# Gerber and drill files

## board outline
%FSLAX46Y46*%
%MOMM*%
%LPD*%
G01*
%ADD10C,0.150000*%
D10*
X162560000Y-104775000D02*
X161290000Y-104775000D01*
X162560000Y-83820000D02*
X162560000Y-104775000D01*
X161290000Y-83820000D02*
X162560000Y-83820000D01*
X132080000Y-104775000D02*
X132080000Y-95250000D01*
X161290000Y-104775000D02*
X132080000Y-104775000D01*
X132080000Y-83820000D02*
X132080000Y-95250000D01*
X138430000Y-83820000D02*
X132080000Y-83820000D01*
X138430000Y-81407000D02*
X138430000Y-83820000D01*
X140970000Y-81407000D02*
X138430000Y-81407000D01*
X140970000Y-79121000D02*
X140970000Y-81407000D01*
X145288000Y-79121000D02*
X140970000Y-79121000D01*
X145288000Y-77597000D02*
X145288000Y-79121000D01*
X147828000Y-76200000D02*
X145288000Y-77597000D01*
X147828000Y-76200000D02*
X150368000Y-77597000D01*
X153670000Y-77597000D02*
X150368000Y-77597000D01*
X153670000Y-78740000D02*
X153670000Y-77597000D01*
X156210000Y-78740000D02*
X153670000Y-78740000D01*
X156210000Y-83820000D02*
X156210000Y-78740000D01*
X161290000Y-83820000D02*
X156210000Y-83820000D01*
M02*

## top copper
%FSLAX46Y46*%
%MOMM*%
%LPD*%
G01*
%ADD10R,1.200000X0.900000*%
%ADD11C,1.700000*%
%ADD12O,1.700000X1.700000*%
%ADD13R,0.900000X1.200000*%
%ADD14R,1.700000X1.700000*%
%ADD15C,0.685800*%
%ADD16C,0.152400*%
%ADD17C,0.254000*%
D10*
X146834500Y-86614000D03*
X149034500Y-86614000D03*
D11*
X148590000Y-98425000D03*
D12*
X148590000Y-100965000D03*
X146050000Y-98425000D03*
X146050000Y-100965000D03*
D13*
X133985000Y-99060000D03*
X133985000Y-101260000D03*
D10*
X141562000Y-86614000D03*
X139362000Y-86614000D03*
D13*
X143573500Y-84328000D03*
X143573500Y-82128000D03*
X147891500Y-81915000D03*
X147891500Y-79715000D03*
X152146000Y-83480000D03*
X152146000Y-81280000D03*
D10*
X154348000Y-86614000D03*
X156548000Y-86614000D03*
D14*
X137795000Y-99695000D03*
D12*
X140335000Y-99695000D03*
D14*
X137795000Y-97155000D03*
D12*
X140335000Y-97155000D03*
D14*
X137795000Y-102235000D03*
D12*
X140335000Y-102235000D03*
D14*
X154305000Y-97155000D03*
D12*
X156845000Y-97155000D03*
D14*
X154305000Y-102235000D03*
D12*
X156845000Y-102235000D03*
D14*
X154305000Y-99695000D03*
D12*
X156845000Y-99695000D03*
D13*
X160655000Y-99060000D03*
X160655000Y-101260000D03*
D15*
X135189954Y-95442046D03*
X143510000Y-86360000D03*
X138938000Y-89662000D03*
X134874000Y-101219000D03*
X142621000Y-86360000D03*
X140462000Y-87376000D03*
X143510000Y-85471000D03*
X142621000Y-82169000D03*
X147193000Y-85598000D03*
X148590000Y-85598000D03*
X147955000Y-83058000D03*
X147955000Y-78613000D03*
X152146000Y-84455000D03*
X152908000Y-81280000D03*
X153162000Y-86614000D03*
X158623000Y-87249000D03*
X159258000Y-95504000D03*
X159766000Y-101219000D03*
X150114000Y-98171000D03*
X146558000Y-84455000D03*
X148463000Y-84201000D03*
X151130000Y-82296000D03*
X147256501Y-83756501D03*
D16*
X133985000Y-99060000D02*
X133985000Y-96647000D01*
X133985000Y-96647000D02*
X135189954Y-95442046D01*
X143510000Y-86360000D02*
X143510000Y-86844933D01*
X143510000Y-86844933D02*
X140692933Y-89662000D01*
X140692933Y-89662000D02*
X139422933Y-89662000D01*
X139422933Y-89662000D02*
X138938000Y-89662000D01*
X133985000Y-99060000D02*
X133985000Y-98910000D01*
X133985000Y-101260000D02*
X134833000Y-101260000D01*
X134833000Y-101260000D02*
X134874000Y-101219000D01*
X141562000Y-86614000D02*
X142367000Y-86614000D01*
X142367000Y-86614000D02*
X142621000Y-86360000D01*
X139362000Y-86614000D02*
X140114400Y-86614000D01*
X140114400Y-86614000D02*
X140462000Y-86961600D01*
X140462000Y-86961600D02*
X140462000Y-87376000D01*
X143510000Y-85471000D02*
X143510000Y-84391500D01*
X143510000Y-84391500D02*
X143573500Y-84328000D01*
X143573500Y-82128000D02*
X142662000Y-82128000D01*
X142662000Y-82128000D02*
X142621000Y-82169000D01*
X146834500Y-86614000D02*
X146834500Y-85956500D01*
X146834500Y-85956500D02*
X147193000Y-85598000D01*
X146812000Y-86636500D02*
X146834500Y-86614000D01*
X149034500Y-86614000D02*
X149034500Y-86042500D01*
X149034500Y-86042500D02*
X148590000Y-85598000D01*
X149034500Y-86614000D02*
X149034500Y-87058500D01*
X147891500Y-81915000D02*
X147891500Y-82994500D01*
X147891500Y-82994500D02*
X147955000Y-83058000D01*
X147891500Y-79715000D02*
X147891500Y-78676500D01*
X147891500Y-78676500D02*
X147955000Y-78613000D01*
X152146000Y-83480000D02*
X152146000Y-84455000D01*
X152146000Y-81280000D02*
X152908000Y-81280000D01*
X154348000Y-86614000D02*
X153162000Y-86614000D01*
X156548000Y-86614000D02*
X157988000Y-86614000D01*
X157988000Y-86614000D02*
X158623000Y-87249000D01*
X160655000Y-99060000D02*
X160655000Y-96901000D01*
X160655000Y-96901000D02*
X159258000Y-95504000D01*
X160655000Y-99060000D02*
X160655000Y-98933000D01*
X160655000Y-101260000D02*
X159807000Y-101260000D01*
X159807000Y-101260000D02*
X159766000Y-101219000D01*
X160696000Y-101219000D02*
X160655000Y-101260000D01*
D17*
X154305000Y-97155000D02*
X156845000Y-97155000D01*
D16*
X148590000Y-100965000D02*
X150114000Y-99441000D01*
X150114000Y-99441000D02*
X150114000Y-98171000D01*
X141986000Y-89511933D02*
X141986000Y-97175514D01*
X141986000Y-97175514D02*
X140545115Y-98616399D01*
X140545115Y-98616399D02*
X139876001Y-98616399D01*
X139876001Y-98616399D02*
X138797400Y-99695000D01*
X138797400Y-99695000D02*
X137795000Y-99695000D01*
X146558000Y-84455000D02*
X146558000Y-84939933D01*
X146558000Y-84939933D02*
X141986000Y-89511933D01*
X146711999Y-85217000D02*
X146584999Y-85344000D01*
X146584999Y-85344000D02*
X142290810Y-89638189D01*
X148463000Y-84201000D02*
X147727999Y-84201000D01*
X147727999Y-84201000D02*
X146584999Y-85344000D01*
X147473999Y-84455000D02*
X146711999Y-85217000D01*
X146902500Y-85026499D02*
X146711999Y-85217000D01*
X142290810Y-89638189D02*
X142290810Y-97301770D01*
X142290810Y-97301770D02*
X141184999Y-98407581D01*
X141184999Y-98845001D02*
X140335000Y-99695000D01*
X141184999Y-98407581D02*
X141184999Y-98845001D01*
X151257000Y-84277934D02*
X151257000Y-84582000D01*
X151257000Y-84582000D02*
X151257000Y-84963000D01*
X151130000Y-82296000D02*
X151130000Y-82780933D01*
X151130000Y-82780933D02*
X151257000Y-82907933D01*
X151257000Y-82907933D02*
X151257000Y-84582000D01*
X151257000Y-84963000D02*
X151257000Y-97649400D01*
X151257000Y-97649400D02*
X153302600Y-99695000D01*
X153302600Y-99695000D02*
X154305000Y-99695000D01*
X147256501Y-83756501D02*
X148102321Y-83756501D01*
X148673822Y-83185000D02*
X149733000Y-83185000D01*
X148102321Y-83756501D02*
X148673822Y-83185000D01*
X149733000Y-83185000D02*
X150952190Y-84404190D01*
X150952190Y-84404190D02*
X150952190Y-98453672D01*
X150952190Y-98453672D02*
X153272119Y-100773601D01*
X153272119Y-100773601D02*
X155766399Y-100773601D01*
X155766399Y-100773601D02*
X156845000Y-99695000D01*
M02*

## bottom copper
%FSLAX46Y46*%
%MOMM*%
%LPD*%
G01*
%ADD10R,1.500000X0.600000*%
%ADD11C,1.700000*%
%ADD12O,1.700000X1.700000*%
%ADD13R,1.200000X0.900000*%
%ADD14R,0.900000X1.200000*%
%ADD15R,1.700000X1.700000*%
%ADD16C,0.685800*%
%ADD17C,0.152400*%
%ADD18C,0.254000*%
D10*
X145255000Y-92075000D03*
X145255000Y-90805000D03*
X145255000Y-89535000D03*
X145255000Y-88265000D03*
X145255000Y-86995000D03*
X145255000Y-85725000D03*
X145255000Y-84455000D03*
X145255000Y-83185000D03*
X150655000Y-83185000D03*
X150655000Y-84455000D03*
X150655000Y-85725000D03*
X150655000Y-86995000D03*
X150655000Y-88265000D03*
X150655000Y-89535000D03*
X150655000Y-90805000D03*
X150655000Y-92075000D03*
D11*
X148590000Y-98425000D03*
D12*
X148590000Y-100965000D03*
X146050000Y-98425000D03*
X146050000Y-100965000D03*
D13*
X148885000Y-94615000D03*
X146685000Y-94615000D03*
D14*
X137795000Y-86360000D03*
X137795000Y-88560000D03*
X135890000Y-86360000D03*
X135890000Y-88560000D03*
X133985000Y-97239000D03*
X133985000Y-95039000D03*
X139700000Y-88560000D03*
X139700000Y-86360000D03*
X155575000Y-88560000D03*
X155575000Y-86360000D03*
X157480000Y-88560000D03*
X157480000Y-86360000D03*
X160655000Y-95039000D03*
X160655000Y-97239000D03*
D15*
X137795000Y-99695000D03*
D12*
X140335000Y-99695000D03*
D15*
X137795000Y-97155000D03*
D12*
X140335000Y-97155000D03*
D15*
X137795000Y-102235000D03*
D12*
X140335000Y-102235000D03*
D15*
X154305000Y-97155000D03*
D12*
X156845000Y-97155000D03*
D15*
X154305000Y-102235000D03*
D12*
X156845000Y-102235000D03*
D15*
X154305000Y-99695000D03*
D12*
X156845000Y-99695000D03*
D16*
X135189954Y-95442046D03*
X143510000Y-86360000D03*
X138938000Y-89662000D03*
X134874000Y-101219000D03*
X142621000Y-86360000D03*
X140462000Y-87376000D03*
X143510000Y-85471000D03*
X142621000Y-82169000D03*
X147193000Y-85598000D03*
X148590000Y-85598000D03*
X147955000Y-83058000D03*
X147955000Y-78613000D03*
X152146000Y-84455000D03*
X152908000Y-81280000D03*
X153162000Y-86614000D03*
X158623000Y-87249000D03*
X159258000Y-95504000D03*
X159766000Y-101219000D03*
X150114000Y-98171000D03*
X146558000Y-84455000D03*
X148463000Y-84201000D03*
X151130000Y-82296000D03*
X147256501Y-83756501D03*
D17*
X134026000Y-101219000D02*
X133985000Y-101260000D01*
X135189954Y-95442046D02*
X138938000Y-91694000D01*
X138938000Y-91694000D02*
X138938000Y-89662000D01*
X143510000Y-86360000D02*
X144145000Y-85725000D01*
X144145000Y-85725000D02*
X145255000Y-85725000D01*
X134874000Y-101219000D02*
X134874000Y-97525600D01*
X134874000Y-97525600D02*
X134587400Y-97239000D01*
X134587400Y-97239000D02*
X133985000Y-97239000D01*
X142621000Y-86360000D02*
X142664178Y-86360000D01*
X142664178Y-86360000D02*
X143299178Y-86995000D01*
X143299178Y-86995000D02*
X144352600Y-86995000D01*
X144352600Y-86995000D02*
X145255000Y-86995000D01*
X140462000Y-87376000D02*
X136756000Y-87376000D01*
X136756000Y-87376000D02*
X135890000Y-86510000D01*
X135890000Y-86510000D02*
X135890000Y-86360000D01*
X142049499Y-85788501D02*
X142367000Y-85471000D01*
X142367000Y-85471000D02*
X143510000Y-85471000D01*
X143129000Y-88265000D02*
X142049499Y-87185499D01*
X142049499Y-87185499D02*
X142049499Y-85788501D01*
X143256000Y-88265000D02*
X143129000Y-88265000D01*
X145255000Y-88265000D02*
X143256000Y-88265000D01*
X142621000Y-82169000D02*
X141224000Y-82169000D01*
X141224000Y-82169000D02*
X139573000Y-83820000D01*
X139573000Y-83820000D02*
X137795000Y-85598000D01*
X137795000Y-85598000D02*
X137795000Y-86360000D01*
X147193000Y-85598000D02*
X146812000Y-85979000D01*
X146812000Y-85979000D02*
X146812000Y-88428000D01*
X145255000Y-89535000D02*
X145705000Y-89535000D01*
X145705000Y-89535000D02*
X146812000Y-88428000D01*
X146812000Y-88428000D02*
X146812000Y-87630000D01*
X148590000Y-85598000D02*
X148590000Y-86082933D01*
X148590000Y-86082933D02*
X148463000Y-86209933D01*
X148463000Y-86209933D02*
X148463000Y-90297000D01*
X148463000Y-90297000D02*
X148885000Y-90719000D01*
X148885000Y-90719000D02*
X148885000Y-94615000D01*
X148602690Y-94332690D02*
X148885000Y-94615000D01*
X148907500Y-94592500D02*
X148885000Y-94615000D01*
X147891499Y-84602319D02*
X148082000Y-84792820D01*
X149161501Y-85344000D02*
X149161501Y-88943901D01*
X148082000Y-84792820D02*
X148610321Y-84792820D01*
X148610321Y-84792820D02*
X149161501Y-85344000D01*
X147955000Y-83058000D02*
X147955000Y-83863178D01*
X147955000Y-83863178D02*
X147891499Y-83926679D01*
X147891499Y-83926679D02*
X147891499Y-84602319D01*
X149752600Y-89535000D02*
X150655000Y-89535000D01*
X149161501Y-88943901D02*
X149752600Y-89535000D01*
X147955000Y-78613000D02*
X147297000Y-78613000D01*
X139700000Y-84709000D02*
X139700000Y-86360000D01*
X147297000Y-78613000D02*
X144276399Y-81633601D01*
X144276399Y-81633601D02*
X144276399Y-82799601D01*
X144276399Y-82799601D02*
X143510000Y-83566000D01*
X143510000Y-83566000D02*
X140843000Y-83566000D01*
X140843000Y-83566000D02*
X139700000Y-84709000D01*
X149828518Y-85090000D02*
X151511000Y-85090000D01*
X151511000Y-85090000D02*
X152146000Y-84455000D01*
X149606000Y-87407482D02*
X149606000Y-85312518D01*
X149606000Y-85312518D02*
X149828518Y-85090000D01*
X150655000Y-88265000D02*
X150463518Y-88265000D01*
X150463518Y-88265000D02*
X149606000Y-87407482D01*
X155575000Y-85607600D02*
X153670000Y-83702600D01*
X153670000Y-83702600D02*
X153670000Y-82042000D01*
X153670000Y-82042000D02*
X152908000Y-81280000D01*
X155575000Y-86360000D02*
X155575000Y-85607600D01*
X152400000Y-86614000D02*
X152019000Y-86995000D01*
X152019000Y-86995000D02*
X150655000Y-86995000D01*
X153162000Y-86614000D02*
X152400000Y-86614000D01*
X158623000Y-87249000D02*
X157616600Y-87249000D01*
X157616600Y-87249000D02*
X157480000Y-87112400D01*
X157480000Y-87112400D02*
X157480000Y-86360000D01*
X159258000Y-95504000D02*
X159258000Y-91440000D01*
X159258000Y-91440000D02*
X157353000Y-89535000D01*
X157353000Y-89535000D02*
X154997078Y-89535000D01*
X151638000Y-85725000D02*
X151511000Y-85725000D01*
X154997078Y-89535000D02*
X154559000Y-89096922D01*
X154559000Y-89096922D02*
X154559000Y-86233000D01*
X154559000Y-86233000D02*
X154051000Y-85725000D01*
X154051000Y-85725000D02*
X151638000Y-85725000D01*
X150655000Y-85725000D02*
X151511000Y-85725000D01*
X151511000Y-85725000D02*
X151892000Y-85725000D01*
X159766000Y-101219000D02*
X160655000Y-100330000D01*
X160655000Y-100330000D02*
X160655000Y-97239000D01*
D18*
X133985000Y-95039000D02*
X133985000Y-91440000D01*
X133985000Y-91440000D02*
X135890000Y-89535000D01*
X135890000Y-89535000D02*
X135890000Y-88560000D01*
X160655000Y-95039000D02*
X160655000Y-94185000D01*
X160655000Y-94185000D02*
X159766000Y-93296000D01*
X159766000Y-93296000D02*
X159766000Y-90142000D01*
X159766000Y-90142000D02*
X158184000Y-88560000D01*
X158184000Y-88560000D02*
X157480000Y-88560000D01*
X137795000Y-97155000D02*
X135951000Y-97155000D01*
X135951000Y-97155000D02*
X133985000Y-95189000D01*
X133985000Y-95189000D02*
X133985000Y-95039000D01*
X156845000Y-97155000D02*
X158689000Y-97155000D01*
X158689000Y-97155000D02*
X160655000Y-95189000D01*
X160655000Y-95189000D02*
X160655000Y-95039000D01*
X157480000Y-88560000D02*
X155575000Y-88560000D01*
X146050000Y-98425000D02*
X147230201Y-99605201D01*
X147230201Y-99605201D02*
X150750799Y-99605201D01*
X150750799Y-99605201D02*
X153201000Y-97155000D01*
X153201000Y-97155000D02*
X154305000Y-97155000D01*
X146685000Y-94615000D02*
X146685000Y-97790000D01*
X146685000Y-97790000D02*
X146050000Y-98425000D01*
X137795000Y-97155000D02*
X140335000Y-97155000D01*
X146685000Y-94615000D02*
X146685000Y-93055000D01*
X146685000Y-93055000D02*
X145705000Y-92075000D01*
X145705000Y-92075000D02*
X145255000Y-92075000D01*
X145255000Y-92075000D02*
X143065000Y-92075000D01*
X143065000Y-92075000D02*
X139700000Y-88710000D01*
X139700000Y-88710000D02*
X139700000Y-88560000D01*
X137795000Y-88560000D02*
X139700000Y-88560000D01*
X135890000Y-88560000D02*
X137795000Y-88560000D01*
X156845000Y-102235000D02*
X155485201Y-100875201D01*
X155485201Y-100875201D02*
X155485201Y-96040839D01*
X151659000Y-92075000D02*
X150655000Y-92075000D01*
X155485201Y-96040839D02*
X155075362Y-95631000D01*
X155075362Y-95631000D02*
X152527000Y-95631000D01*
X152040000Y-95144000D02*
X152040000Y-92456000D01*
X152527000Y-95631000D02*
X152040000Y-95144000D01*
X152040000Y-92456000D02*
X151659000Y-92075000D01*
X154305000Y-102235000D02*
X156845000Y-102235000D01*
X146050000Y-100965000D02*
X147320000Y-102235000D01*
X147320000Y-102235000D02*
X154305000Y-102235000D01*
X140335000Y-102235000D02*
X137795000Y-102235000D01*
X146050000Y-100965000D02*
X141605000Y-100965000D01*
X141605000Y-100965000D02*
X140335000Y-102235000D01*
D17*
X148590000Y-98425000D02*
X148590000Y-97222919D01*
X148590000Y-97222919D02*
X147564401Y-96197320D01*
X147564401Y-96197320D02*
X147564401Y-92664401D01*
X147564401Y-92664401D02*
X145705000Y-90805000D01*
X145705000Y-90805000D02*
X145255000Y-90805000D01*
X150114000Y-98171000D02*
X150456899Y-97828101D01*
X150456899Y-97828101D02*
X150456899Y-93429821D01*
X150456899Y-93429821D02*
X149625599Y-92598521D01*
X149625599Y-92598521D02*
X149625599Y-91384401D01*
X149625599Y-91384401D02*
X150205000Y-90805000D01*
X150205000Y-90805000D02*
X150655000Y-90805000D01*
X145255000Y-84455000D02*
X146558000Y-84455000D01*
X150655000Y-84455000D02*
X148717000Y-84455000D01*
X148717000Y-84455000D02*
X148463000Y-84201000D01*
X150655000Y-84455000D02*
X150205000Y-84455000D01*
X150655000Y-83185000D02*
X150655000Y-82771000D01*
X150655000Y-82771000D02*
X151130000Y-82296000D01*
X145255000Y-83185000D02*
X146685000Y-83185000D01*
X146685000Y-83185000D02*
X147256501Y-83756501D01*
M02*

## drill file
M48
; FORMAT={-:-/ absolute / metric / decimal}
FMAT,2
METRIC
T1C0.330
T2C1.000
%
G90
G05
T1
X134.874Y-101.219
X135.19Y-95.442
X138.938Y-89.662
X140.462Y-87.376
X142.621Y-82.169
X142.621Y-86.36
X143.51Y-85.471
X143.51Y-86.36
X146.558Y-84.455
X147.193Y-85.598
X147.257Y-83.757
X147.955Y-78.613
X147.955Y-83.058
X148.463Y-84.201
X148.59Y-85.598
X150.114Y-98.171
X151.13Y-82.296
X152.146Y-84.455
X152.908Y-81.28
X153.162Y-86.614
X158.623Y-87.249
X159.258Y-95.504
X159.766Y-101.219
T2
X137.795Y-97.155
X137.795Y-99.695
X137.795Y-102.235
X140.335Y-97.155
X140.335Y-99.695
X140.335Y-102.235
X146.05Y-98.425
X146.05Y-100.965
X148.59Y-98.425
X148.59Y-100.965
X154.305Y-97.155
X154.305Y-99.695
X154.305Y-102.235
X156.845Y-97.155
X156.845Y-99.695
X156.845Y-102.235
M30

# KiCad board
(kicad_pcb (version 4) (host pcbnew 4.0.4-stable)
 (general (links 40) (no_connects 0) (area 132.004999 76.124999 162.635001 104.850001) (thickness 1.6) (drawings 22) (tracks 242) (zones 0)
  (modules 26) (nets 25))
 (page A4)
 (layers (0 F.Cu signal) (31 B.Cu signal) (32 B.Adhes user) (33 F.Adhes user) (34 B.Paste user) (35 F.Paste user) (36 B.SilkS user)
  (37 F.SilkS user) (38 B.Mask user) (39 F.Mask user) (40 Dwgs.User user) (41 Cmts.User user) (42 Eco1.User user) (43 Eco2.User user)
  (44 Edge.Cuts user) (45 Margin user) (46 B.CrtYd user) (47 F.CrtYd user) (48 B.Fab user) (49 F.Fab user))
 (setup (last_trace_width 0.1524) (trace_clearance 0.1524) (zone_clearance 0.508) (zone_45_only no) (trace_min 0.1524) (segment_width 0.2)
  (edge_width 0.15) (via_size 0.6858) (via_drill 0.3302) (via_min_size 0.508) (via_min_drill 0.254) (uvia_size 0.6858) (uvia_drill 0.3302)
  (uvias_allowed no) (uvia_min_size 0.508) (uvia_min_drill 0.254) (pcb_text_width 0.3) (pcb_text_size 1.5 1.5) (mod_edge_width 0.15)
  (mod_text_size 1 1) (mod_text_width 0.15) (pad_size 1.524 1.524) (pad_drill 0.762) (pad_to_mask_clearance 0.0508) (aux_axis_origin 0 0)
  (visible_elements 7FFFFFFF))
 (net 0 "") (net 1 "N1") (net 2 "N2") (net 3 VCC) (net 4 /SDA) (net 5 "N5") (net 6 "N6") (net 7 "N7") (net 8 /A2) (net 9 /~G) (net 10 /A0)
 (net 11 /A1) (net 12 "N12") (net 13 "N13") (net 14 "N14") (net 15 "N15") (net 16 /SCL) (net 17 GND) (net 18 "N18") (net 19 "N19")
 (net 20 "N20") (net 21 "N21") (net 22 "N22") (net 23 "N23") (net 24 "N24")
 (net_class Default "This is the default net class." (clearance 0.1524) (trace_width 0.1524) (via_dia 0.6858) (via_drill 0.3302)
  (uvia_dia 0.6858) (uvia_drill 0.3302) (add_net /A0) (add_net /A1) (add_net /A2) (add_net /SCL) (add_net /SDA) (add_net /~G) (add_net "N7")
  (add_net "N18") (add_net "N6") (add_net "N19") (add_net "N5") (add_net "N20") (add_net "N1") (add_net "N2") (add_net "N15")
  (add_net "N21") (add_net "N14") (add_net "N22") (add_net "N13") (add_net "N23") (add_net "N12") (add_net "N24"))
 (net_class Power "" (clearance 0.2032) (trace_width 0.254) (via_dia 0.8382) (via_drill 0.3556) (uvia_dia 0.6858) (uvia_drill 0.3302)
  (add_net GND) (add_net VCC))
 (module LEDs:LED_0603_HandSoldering (layer F.Cu) (at 147.9345 86.614)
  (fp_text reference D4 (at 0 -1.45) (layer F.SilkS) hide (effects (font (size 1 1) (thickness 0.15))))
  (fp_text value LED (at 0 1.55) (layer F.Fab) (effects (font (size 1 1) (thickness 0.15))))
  (pad 1 smd rect (at -1.1 0) (size 1.2 0.9) (layers F.Cu F.Paste F.Mask) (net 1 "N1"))
  (pad 2 smd rect (at 1.1 0) (size 1.2 0.9) (layers F.Cu F.Paste F.Mask) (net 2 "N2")))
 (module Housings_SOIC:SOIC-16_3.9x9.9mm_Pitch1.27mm (layer B.Cu) (at 147.955 87.63)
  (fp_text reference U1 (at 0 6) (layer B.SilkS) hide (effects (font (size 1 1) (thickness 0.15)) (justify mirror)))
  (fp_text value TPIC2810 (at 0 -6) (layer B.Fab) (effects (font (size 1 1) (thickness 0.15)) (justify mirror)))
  (pad 1 smd rect (at -2.7 4.445) (size 1.5 0.6) (layers B.Cu B.Paste B.Mask) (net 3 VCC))
  (pad 2 smd rect (at -2.7 3.175) (size 1.5 0.6) (layers B.Cu B.Paste B.Mask) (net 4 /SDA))
  (pad 3 smd rect (at -2.7 1.905) (size 1.5 0.6) (layers B.Cu B.Paste B.Mask) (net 1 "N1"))
  (pad 4 smd rect (at -2.7 0.635) (size 1.5 0.6) (layers B.Cu B.Paste B.Mask) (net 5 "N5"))
  (pad 5 smd rect (at -2.7 -0.635) (size 1.5 0.6) (layers B.Cu B.Paste B.Mask) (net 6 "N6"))
  (pad 6 smd rect (at -2.7 -1.905) (size 1.5 0.6) (layers B.Cu B.Paste B.Mask) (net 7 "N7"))
  (pad 7 smd rect (at -2.7 -3.175) (size 1.5 0.6) (layers B.Cu B.Paste B.Mask) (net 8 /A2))
  (pad 8 smd rect (at -2.7 -4.445) (size 1.5 0.6) (layers B.Cu B.Paste B.Mask) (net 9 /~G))
  (pad 9 smd rect (at 2.7 -4.445) (size 1.5 0.6) (layers B.Cu B.Paste B.Mask) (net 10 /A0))
  (pad 10 smd rect (at 2.7 -3.175) (size 1.5 0.6) (layers B.Cu B.Paste B.Mask) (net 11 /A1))
  (pad 11 smd rect (at 2.7 -1.905) (size 1.5 0.6) (layers B.Cu B.Paste B.Mask) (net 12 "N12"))
  (pad 12 smd rect (at 2.7 -0.635) (size 1.5 0.6) (layers B.Cu B.Paste B.Mask) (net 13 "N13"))
  (pad 13 smd rect (at 2.7 0.635) (size 1.5 0.6) (layers B.Cu B.Paste B.Mask) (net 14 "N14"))
  (pad 14 smd rect (at 2.7 1.905) (size 1.5 0.6) (layers B.Cu B.Paste B.Mask) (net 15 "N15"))
  (pad 15 smd rect (at 2.7 3.175) (size 1.5 0.6) (layers B.Cu B.Paste B.Mask) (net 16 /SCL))
  (pad 16 smd rect (at 2.7 4.445) (size 1.5 0.6) (layers B.Cu B.Paste B.Mask) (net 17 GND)))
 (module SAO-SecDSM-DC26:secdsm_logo (layer F.Cu) (at 147.32 85.979)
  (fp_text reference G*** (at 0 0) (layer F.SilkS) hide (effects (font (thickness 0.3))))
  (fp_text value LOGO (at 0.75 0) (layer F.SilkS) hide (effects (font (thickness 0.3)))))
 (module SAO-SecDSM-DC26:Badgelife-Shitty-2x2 (layer F.Cu) (at 147.32 99.695)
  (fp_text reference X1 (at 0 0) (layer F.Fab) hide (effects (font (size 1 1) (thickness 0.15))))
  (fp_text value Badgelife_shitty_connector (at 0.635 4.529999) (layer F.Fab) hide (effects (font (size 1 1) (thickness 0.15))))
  (pad 4 thru_hole circle (at 1.27 -1.27) (size 1.7 1.7) (drill 1) (layers *.Cu *.Mask) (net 4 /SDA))
  (pad 3 thru_hole oval (at 1.27 1.27) (size 1.7 1.7) (drill 1) (layers *.Cu *.Mask) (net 16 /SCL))
  (pad 1 thru_hole oval (at -1.27 -1.27) (size 1.7 1.7) (drill 1) (layers *.Cu *.Mask) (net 3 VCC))
  (pad 2 thru_hole oval (at -1.27 1.27) (size 1.7 1.7) (drill 1) (layers *.Cu *.Mask) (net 17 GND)))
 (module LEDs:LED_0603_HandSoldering (layer F.Cu) (at 133.985 100.16 270)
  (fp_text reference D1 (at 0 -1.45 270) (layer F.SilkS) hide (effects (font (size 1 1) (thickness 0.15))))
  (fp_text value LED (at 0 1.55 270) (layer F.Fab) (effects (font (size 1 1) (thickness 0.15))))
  (pad 1 smd rect (at -1.1 0 270) (size 1.2 0.9) (layers F.Cu F.Paste F.Mask) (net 7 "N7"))
  (pad 2 smd rect (at 1.1 0 270) (size 1.2 0.9) (layers F.Cu F.Paste F.Mask) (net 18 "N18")))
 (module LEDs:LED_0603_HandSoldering (layer F.Cu) (at 140.462 86.614 180)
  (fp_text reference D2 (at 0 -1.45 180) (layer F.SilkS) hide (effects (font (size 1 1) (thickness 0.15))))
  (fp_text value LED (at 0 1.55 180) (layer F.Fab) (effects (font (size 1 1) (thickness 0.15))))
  (pad 1 smd rect (at -1.1 0 180) (size 1.2 0.9) (layers F.Cu F.Paste F.Mask) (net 6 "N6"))
  (pad 2 smd rect (at 1.1 0 180) (size 1.2 0.9) (layers F.Cu F.Paste F.Mask) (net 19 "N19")))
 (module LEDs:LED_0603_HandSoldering (layer F.Cu) (at 143.5735 83.228 90)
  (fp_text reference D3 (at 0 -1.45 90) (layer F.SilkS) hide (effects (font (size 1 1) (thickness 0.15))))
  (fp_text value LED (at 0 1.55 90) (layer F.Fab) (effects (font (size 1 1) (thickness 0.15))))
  (pad 1 smd rect (at -1.1 0 90) (size 1.2 0.9) (layers F.Cu F.Paste F.Mask) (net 5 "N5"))
  (pad 2 smd rect (at 1.1 0 90) (size 1.2 0.9) (layers F.Cu F.Paste F.Mask) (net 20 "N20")))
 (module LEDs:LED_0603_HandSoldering (layer F.Cu) (at 147.8915 80.815 90)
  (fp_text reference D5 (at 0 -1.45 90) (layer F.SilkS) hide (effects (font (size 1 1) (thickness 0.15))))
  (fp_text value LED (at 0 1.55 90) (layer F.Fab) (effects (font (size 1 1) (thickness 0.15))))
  (pad 1 smd rect (at -1.1 0 90) (size 1.2 0.9) (layers F.Cu F.Paste F.Mask) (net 15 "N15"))
  (pad 2 smd rect (at 1.1 0 90) (size 1.2 0.9) (layers F.Cu F.Paste F.Mask) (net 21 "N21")))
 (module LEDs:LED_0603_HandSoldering (layer F.Cu) (at 152.146 82.38 90)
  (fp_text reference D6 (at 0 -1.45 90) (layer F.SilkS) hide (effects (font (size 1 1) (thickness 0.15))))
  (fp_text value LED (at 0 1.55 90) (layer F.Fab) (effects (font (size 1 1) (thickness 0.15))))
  (pad 1 smd rect (at -1.1 0 90) (size 1.2 0.9) (layers F.Cu F.Paste F.Mask) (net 14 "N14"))
  (pad 2 smd rect (at 1.1 0 90) (size 1.2 0.9) (layers F.Cu F.Paste F.Mask) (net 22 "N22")))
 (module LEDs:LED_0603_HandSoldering (layer F.Cu) (at 155.448 86.614)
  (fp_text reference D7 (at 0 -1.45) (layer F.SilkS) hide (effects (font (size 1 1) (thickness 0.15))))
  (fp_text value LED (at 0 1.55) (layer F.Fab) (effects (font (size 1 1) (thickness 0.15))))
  (pad 1 smd rect (at -1.1 0) (size 1.2 0.9) (layers F.Cu F.Paste F.Mask) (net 13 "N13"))
  (pad 2 smd rect (at 1.1 0) (size 1.2 0.9) (layers F.Cu F.Paste F.Mask) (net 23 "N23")))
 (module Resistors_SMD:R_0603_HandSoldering (layer B.Cu) (at 147.785 94.615 180)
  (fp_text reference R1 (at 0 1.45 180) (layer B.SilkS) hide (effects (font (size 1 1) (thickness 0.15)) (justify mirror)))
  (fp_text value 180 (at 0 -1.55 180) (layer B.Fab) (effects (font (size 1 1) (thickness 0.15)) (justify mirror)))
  (pad 1 smd rect (at -1.1 0 180) (size 1.2 0.9) (layers B.Cu B.Paste B.Mask) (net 2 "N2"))
  (pad 2 smd rect (at 1.1 0 180) (size 1.2 0.9) (layers B.Cu B.Paste B.Mask) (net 3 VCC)))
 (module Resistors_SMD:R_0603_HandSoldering (layer B.Cu) (at 137.795 87.46 270)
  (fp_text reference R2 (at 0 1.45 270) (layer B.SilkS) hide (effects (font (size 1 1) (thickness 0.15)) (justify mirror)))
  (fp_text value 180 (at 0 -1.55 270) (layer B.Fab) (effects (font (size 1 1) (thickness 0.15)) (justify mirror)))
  (pad 1 smd rect (at -1.1 0 270) (size 1.2 0.9) (layers B.Cu B.Paste B.Mask) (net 20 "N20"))
  (pad 2 smd rect (at 1.1 0 270) (size 1.2 0.9) (layers B.Cu B.Paste B.Mask) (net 3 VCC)))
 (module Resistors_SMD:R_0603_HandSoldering (layer B.Cu) (at 135.89 87.46 270)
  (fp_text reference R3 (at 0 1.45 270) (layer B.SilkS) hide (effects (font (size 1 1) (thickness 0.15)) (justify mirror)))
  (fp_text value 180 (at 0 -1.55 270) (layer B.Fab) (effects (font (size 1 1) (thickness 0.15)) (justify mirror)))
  (pad 1 smd rect (at -1.1 0 270) (size 1.2 0.9) (layers B.Cu B.Paste B.Mask) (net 19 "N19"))
  (pad 2 smd rect (at 1.1 0 270) (size 1.2 0.9) (layers B.Cu B.Paste B.Mask) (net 3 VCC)))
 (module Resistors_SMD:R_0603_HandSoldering (layer B.Cu) (at 133.985 96.139 90)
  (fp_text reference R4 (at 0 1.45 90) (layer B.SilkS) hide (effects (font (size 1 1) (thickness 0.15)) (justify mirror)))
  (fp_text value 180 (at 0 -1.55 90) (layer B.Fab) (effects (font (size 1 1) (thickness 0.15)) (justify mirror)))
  (pad 1 smd rect (at -1.1 0 90) (size 1.2 0.9) (layers B.Cu B.Paste B.Mask) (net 18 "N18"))
  (pad 2 smd rect (at 1.1 0 90) (size 1.2 0.9) (layers B.Cu B.Paste B.Mask) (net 3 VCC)))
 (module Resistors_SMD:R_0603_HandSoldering (layer B.Cu) (at 139.7 87.46 90)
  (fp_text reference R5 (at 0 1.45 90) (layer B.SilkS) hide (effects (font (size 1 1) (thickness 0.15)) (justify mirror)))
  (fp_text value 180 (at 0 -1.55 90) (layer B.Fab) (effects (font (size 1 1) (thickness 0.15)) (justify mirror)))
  (pad 1 smd rect (at -1.1 0 90) (size 1.2 0.9) (layers B.Cu B.Paste B.Mask) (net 3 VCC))
  (pad 2 smd rect (at 1.1 0 90) (size 1.2 0.9) (layers B.Cu B.Paste B.Mask) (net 21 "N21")))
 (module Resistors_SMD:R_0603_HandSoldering (layer B.Cu) (at 155.575 87.46 90)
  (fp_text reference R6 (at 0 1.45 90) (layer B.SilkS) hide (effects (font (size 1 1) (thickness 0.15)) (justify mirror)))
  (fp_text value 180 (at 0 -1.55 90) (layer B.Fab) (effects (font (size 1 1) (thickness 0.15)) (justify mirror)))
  (pad 1 smd rect (at -1.1 0 90) (size 1.2 0.9) (layers B.Cu B.Paste B.Mask) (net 3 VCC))
  (pad 2 smd rect (at 1.1 0 90) (size 1.2 0.9) (layers B.Cu B.Paste B.Mask) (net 22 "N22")))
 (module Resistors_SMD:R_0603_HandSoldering (layer B.Cu) (at 157.48 87.46 90)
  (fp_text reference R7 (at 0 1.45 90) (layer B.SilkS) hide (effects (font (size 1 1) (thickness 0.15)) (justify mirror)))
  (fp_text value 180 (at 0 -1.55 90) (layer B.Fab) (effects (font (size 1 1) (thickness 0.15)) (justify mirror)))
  (pad 1 smd rect (at -1.1 0 90) (size 1.2 0.9) (layers B.Cu B.Paste B.Mask) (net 3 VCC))
  (pad 2 smd rect (at 1.1 0 90) (size 1.2 0.9) (layers B.Cu B.Paste B.Mask) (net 23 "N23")))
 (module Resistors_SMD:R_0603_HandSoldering (layer B.Cu) (at 160.655 96.139 270)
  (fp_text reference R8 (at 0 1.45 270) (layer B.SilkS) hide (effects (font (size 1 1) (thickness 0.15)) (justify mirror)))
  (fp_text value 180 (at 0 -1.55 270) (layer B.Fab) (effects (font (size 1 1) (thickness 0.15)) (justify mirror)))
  (pad 1 smd rect (at -1.1 0 270) (size 1.2 0.9) (layers B.Cu B.Paste B.Mask) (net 3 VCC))
  (pad 2 smd rect (at 1.1 0 270) (size 1.2 0.9) (layers B.Cu B.Paste B.Mask) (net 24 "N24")))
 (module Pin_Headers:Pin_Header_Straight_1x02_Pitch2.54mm (layer F.Cu) (at 137.795 99.695 90)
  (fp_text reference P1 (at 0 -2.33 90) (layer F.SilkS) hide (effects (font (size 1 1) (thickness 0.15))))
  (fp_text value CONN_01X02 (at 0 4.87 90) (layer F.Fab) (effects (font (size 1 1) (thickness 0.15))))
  (pad 1 thru_hole rect (at 0 0 90) (size 1.7 1.7) (drill 1) (layers *.Cu *.Mask) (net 8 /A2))
  (pad 2 thru_hole oval (at 0 2.54 90) (size 1.7 1.7) (drill 1) (layers *.Cu *.Mask) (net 11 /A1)))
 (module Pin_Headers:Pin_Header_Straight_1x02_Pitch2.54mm (layer F.Cu) (at 137.795 97.155 90)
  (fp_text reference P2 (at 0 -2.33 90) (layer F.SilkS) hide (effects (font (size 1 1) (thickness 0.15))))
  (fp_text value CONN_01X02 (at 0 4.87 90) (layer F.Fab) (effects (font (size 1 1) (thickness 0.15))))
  (pad 1 thru_hole rect (at 0 0 90) (size 1.7 1.7) (drill 1) (layers *.Cu *.Mask) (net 3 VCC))
  (pad 2 thru_hole oval (at 0 2.54 90) (size 1.7 1.7) (drill 1) (layers *.Cu *.Mask) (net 3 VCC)))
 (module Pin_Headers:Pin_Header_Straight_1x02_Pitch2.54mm (layer F.Cu) (at 137.795 102.235 90)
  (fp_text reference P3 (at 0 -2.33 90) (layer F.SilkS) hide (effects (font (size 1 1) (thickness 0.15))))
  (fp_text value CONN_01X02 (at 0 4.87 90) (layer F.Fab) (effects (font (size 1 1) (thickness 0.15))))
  (pad 1 thru_hole rect (at 0 0 90) (size 1.7 1.7) (drill 1) (layers *.Cu *.Mask) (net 17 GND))
  (pad 2 thru_hole oval (at 0 2.54 90) (size 1.7 1.7) (drill 1) (layers *.Cu *.Mask) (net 17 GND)))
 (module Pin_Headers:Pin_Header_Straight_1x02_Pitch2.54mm (layer F.Cu) (at 154.305 97.155 90)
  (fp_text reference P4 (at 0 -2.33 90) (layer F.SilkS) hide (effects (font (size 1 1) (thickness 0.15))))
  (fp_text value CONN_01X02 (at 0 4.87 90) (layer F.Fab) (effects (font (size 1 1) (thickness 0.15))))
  (pad 1 thru_hole rect (at 0 0 90) (size 1.7 1.7) (drill 1) (layers *.Cu *.Mask) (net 3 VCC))
  (pad 2 thru_hole oval (at 0 2.54 90) (size 1.7 1.7) (drill 1) (layers *.Cu *.Mask) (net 3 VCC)))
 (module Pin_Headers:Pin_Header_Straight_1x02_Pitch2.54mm (layer F.Cu) (at 154.305 102.235 90)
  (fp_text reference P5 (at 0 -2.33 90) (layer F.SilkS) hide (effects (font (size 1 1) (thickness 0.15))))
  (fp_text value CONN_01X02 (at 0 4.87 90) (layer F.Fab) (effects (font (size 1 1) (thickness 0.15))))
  (pad 1 thru_hole rect (at 0 0 90) (size 1.7 1.7) (drill 1) (layers *.Cu *.Mask) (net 17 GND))
  (pad 2 thru_hole oval (at 0 2.54 90) (size 1.7 1.7) (drill 1) (layers *.Cu *.Mask) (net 17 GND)))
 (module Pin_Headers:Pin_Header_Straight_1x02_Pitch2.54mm (layer F.Cu) (at 154.305 99.695 90)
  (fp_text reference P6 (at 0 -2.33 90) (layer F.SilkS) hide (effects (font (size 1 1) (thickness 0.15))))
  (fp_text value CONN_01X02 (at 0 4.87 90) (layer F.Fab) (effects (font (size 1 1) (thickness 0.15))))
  (pad 1 thru_hole rect (at 0 0 90) (size 1.7 1.7) (drill 1) (layers *.Cu *.Mask) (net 10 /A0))
  (pad 2 thru_hole oval (at 0 2.54 90) (size 1.7 1.7) (drill 1) (layers *.Cu *.Mask) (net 9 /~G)))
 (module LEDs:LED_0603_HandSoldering (layer F.Cu) (at 160.655 100.16 270)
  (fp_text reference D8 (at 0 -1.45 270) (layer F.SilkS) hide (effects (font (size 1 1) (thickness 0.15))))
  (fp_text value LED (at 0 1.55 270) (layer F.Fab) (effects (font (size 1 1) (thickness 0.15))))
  (pad 1 smd rect (at -1.1 0 270) (size 1.2 0.9) (layers F.Cu F.Paste F.Mask) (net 12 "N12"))
  (pad 2 smd rect (at 1.1 0 270) (size 1.2 0.9) (layers F.Cu F.Paste F.Mask) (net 24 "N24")))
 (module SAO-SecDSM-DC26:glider (layer B.Cu) (at 155.575 92.583 180)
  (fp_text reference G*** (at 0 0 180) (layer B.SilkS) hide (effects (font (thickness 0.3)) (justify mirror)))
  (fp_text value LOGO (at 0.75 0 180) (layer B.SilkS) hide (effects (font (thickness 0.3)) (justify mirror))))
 (gr_line (start 162.56 104.775) (end 161.29 104.775) (layer Edge.Cuts) (width 0.15))
 (gr_line (start 162.56 83.82) (end 162.56 104.775) (layer Edge.Cuts) (width 0.15))
 (gr_line (start 161.29 83.82) (end 162.56 83.82) (layer Edge.Cuts) (width 0.15))
 (gr_line (start 132.08 104.775) (end 132.08 95.25) (layer Edge.Cuts) (width 0.15))
 (gr_line (start 161.29 104.775) (end 132.08 104.775) (layer Edge.Cuts) (width 0.15))
 (gr_line (start 132.08 83.82) (end 132.08 95.25) (layer Edge.Cuts) (width 0.15))
 (gr_line (start 138.43 83.82) (end 132.08 83.82) (layer Edge.Cuts) (width 0.15))
 (gr_line (start 138.43 81.407) (end 138.43 83.82) (layer Edge.Cuts) (width 0.15))
 (gr_line (start 140.97 81.407) (end 138.43 81.407) (layer Edge.Cuts) (width 0.15))
 (gr_line (start 140.97 79.121) (end 140.97 81.407) (layer Edge.Cuts) (width 0.15))
 (gr_line (start 145.288 79.121) (end 140.97 79.121) (layer Edge.Cuts) (width 0.15))
 (gr_line (start 145.288 77.597) (end 145.288 79.121) (layer Edge.Cuts) (width 0.15))
 (gr_line (start 147.828 76.2) (end 145.288 77.597) (layer Edge.Cuts) (width 0.15))
 (gr_line (start 147.828 76.2) (end 150.368 77.597) (layer Edge.Cuts) (width 0.15))
 (gr_line (start 153.67 77.597) (end 150.368 77.597) (layer Edge.Cuts) (width 0.15))
 (gr_line (start 153.67 78.74) (end 153.67 77.597) (layer Edge.Cuts) (width 0.15))
 (gr_line (start 156.21 78.74) (end 153.67 78.74) (layer Edge.Cuts) (width 0.15))
 (gr_line (start 156.21 83.82) (end 156.21 78.74) (layer Edge.Cuts) (width 0.15))
 (gr_line (start 161.29 83.82) (end 156.21 83.82) (layer Edge.Cuts) (width 0.15))
 (segment (start 134.026 101.219) (end 133.985 101.26) (width 0.1524) (layer B.Cu) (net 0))
 (segment (start 135.189954 95.442046) (end 138.938 91.694) (width 0.1524) (layer B.Cu) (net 7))
 (segment (start 138.938 91.694) (end 138.938 89.662) (width 0.1524) (layer B.Cu) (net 7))
 (segment (start 133.985 99.06) (end 133.985 96.647) (width 0.1524) (layer F.Cu) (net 7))
 (segment (start 133.985 96.647) (end 135.189954 95.442046) (width 0.1524) (layer F.Cu) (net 7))
 (via (at 135.189954 95.442046) (size 0.6858) (drill 0.3302) (layers F.Cu B.Cu) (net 7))
 (segment (start 143.51 86.36) (end 143.51 86.844933) (width 0.1524) (layer F.Cu) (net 7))
 (segment (start 143.51 86.844933) (end 140.692933 89.662) (width 0.1524) (layer F.Cu) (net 7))
 (segment (start 140.692933 89.662) (end 139.422933 89.662) (width 0.1524) (layer F.Cu) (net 7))
 (segment (start 139.422933 89.662) (end 138.938 89.662) (width 0.1524) (layer F.Cu) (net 7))
 (segment (start 143.51 86.36) (end 144.145 85.725) (width 0.1524) (layer B.Cu) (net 7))
 (segment (start 144.145 85.725) (end 145.255 85.725) (width 0.1524) (layer B.Cu) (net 7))
 (via (at 143.51 86.36) (size 0.6858) (drill 0.3302) (layers F.Cu B.Cu) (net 7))
 (via (at 138.938 89.662) (size 0.6858) (drill 0.3302) (layers F.Cu B.Cu) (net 7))
 (segment (start 133.985 99.06) (end 133.985 98.91) (width 0.1524) (layer F.Cu) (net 7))
 (segment (start 134.874 101.219) (end 134.874 97.5256) (width 0.1524) (layer B.Cu) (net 18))
 (segment (start 134.874 97.5256) (end 134.5874 97.239) (width 0.1524) (layer B.Cu) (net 18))
 (segment (start 134.5874 97.239) (end 133.985 97.239) (width 0.1524) (layer B.Cu) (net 18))
 (segment (start 133.985 101.26) (end 134.833 101.26) (width 0.1524) (layer F.Cu) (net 18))
 (segment (start 134.833 101.26) (end 134.874 101.219) (width 0.1524) (layer F.Cu) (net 18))
 (via (at 134.874 101.219) (size 0.6858) (drill 0.3302) (layers F.Cu B.Cu) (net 18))
 (segment (start 142.621 86.36) (end 142.664178 86.36) (width 0.1524) (layer B.Cu) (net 6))
 (segment (start 142.664178 86.36) (end 143.299178 86.995) (width 0.1524) (layer B.Cu) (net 6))
 (segment (start 143.299178 86.995) (end 144.3526 86.995) (width 0.1524) (layer B.Cu) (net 6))
 (segment (start 144.3526 86.995) (end 145.255 86.995) (width 0.1524) (layer B.Cu) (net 6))
 (segment (start 141.562 86.614) (end 142.367 86.614) (width 0.1524) (layer F.Cu) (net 6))
 (segment (start 142.367 86.614) (end 142.621 86.36) (width 0.1524) (layer F.Cu) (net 6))
 (via (at 142.621 86.36) (size 0.6858) (drill 0.3302) (layers F.Cu B.Cu) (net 6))
 (segment (start 140.462 87.376) (end 136.756 87.376) (width 0.1524) (layer B.Cu) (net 19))
 (segment (start 136.756 87.376) (end 135.89 86.51) (width 0.1524) (layer B.Cu) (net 19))
 (segment (start 135.89 86.51) (end 135.89 86.36) (width 0.1524) (layer B.Cu) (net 19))
 (segment (start 139.362 86.614) (end 140.1144 86.614) (width 0.1524) (layer F.Cu) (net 19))
 (segment (start 140.1144 86.614) (end 140.462 86.9616) (width 0.1524) (layer F.Cu) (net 19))
 (segment (start 140.462 86.9616) (end 140.462 87.376) (width 0.1524) (layer F.Cu) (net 19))
 (via (at 140.462 87.376) (size 0.6858) (drill 0.3302) (layers F.Cu B.Cu) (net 19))
 (segment (start 143.51 85.471) (end 143.51 84.3915) (width 0.1524) (layer F.Cu) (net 5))
 (segment (start 143.51 84.3915) (end 143.5735 84.328) (width 0.1524) (layer F.Cu) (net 5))
 (segment (start 142.049499 85.788501) (end 142.367 85.471) (width 0.1524) (layer B.Cu) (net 5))
 (segment (start 142.367 85.471) (end 143.51 85.471) (width 0.1524) (layer B.Cu) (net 5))
 (via (at 143.51 85.471) (size 0.6858) (drill 0.3302) (layers F.Cu B.Cu) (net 5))
 (segment (start 143.129 88.265) (end 142.049499 87.185499) (width 0.1524) (layer B.Cu) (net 5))
 (segment (start 142.049499 87.185499) (end 142.049499 85.788501) (width 0.1524) (layer B.Cu) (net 5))
 (segment (start 143.256 88.265) (end 143.129 88.265) (width 0.1524) (layer B.Cu) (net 5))
 (segment (start 145.255 88.265) (end 143.256 88.265) (width 0.1524) (layer B.Cu) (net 5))
 (segment (start 142.621 82.169) (end 141.224 82.169) (width 0.1524) (layer B.Cu) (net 20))
 (segment (start 141.224 82.169) (end 139.573 83.82) (width 0.1524) (layer B.Cu) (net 20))
 (segment (start 143.5735 82.128) (end 142.662 82.128) (width 0.1524) (layer F.Cu) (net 20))
 (segment (start 142.662 82.128) (end 142.621 82.169) (width 0.1524) (layer F.Cu) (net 20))
 (via (at 142.621 82.169) (size 0.6858) (drill 0.3302) (layers F.Cu B.Cu) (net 20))
 (segment (start 139.573 83.82) (end 137.795 85.598) (width 0.1524) (layer B.Cu) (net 20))
 (segment (start 137.795 85.598) (end 137.795 86.36) (width 0.1524) (layer B.Cu) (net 20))
 (segment (start 147.193 85.598) (end 146.812 85.979) (width 0.1524) (layer B.Cu) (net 1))
 (segment (start 146.812 85.979) (end 146.812 88.428) (width 0.1524) (layer B.Cu) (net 1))
 (segment (start 146.8345 86.614) (end 146.8345 85.9565) (width 0.1524) (layer F.Cu) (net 1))
 (segment (start 146.8345 85.9565) (end 147.193 85.598) (width 0.1524) (layer F.Cu) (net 1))
 (via (at 147.193 85.598) (size 0.6858) (drill 0.3302) (layers F.Cu B.Cu) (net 1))
 (segment (start 146.812 86.6365) (end 146.8345 86.614) (width 0.1524) (layer F.Cu) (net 1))
 (segment (start 145.255 89.535) (end 145.705 89.535) (width 0.1524) (layer B.Cu) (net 1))
 (segment (start 145.705 89.535) (end 146.812 88.428) (width 0.1524) (layer B.Cu) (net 1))
 (segment (start 146.812 88.428) (end 146.812 87.63) (width 0.1524) (layer B.Cu) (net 1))
 (segment (start 148.59 85.598) (end 148.59 86.082933) (width 0.1524) (layer B.Cu) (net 2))
 (segment (start 148.59 86.082933) (end 148.463 86.209933) (width 0.1524) (layer B.Cu) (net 2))
 (segment (start 148.463 86.209933) (end 148.463 90.297) (width 0.1524) (layer B.Cu) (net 2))
 (segment (start 148.463 90.297) (end 148.885 90.719) (width 0.1524) (layer B.Cu) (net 2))
 (segment (start 148.885 90.719) (end 148.885 94.615) (width 0.1524) (layer B.Cu) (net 2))
 (segment (start 149.0345 86.614) (end 149.0345 86.0425) (width 0.1524) (layer F.Cu) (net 2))
 (segment (start 149.0345 86.0425) (end 148.59 85.598) (width 0.1524) (layer F.Cu) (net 2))
 (via (at 148.59 85.598) (size 0.6858) (drill 0.3302) (layers F.Cu B.Cu) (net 2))
 (segment (start 149.0345 86.614) (end 149.0345 87.0585) (width 0.1524) (layer F.Cu) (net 2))
 (segment (start 148.60269 94.33269) (end 148.885 94.615) (width 0.1524) (layer B.Cu) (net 2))
 (segment (start 148.9075 94.5925) (end 148.885 94.615) (width 0.1524) (layer B.Cu) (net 2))
 (segment (start 147.891499 84.602319) (end 148.082 84.79282) (width 0.1524) (layer B.Cu) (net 15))
 (segment (start 149.161501 85.344) (end 149.161501 88.943901) (width 0.1524) (layer B.Cu) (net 15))
 (segment (start 148.082 84.79282) (end 148.610321 84.79282) (width 0.1524) (layer B.Cu) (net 15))
 (segment (start 148.610321 84.79282) (end 149.161501 85.344) (width 0.1524) (layer B.Cu) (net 15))
 (segment (start 147.955 83.058) (end 147.955 83.863178) (width 0.1524) (layer B.Cu) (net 15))
 (segment (start 147.955 83.863178) (end 147.891499 83.926679) (width 0.1524) (layer B.Cu) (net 15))
 (segment (start 147.891499 83.926679) (end 147.891499 84.602319) (width 0.1524) (layer B.Cu) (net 15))
 (segment (start 149.7526 89.535) (end 150.655 89.535) (width 0.1524) (layer B.Cu) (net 15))
 (segment (start 149.161501 88.943901) (end 149.7526 89.535) (width 0.1524) (layer B.Cu) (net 15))
 (segment (start 147.8915 81.915) (end 147.8915 82.9945) (width 0.1524) (layer F.Cu) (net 15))
 (segment (start 147.8915 82.9945) (end 147.955 83.058) (width 0.1524) (layer F.Cu) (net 15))
 (via (at 147.955 83.058) (size 0.6858) (drill 0.3302) (layers F.Cu B.Cu) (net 15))
 (segment (start 147.955 78.613) (end 147.297 78.613) (width 0.1524) (layer B.Cu) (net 21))
 (segment (start 139.7 84.709) (end 139.7 86.36) (width 0.1524) (layer B.Cu) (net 21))
 (segment (start 147.297 78.613) (end 144.276399 81.633601) (width 0.1524) (layer B.Cu) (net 21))
 (segment (start 144.276399 81.633601) (end 144.276399 82.799601) (width 0.1524) (layer B.Cu) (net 21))
 (segment (start 144.276399 82.799601) (end 143.51 83.566) (width 0.1524) (layer B.Cu) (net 21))
 (segment (start 143.51 83.566) (end 140.843 83.566) (width 0.1524) (layer B.Cu) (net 21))
 (segment (start 140.843 83.566) (end 139.7 84.709) (width 0.1524) (layer B.Cu) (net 21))
 (segment (start 147.8915 79.715) (end 147.8915 78.6765) (width 0.1524) (layer F.Cu) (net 21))
 (segment (start 147.8915 78.6765) (end 147.955 78.613) (width 0.1524) (layer F.Cu) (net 21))
 (via (at 147.955 78.613) (size 0.6858) (drill 0.3302) (layers F.Cu B.Cu) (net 21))
 (segment (start 149.828518 85.09) (end 151.511 85.09) (width 0.1524) (layer B.Cu) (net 14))
 (segment (start 151.511 85.09) (end 152.146 84.455) (width 0.1524) (layer B.Cu) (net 14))
 (segment (start 149.606 87.407482) (end 149.606 85.312518) (width 0.1524) (layer B.Cu) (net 14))
 (segment (start 149.606 85.312518) (end 149.828518 85.09) (width 0.1524) (layer B.Cu) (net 14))
 (segment (start 150.655 88.265) (end 150.463518 88.265) (width 0.1524) (layer B.Cu) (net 14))
 (segment (start 150.463518 88.265) (end 149.606 87.407482) (width 0.1524) (layer B.Cu) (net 14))
 (segment (start 152.146 83.48) (end 152.146 84.455) (width 0.1524) (layer F.Cu) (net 14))
 (via (at 152.146 84.455) (size 0.6858) (drill 0.3302) (layers F.Cu B.Cu) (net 14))
 (segment (start 155.575 85.6076) (end 153.67 83.7026) (width 0.1524) (layer B.Cu) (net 22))
 (segment (start 153.67 83.7026) (end 153.67 82.042) (width 0.1524) (layer B.Cu) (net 22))
 (segment (start 153.67 82.042) (end 152.908 81.28) (width 0.1524) (layer B.Cu) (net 22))
 (segment (start 155.575 86.36) (end 155.575 85.6076) (width 0.1524) (layer B.Cu) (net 22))
 (segment (start 152.146 81.28) (end 152.908 81.28) (width 0.1524) (layer F.Cu) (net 22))
 (via (at 152.908 81.28) (size 0.6858) (drill 0.3302) (layers F.Cu B.Cu) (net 22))
 (segment (start 152.4 86.614) (end 152.019 86.995) (width 0.1524) (layer B.Cu) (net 13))
 (segment (start 152.019 86.995) (end 150.655 86.995) (width 0.1524) (layer B.Cu) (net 13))
 (segment (start 153.162 86.614) (end 152.4 86.614) (width 0.1524) (layer B.Cu) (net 13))
 (segment (start 154.348 86.614) (end 153.162 86.614) (width 0.1524) (layer F.Cu) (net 13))
 (via (at 153.162 86.614) (size 0.6858) (drill 0.3302) (layers F.Cu B.Cu) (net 13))
 (segment (start 158.623 87.249) (end 157.6166 87.249) (width 0.1524) (layer B.Cu) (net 23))
 (segment (start 157.6166 87.249) (end 157.48 87.1124) (width 0.1524) (layer B.Cu) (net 23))
 (segment (start 157.48 87.1124) (end 157.48 86.36) (width 0.1524) (layer B.Cu) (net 23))
 (segment (start 156.548 86.614) (end 157.988 86.614) (width 0.1524) (layer F.Cu) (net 23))
 (segment (start 157.988 86.614) (end 158.623 87.249) (width 0.1524) (layer F.Cu) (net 23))
 (via (at 158.623 87.249) (size 0.6858) (drill 0.3302) (layers F.Cu B.Cu) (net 23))
 (segment (start 159.258 95.504) (end 159.258 91.44) (width 0.1524) (layer B.Cu) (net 12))
 (segment (start 159.258 91.44) (end 157.353 89.535) (width 0.1524) (layer B.Cu) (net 12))
 (segment (start 157.353 89.535) (end 154.997078 89.535) (width 0.1524) (layer B.Cu) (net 12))
 (segment (start 151.638 85.725) (end 151.511 85.725) (width 0.1524) (layer B.Cu) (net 12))
 (segment (start 154.997078 89.535) (end 154.559 89.096922) (width 0.1524) (layer B.Cu) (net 12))
 (segment (start 154.559 89.096922) (end 154.559 86.233) (width 0.1524) (layer B.Cu) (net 12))
 (segment (start 154.559 86.233) (end 154.051 85.725) (width 0.1524) (layer B.Cu) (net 12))
 (segment (start 154.051 85.725) (end 151.638 85.725) (width 0.1524) (layer B.Cu) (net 12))
 (segment (start 150.655 85.725) (end 151.511 85.725) (width 0.1524) (layer B.Cu) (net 12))
 (segment (start 151.511 85.725) (end 151.892 85.725) (width 0.1524) (layer B.Cu) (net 12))
 (segment (start 160.655 99.06) (end 160.655 96.901) (width 0.1524) (layer F.Cu) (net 12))
 (segment (start 160.655 96.901) (end 159.258 95.504) (width 0.1524) (layer F.Cu) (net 12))
 (via (at 159.258 95.504) (size 0.6858) (drill 0.3302) (layers F.Cu B.Cu) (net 12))
 (segment (start 160.655 99.06) (end 160.655 98.933) (width 0.1524) (layer F.Cu) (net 12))
 (segment (start 159.766 101.219) (end 160.655 100.33) (width 0.1524) (layer B.Cu) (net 24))
 (segment (start 160.655 100.33) (end 160.655 97.239) (width 0.1524) (layer B.Cu) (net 24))
 (segment (start 160.655 101.26) (end 159.807 101.26) (width 0.1524) (layer F.Cu) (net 24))
 (segment (start 159.807 101.26) (end 159.766 101.219) (width 0.1524) (layer F.Cu) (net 24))
 (via (at 159.766 101.219) (size 0.6858) (drill 0.3302) (layers F.Cu B.Cu) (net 24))
 (segment (start 160.696 101.219) (end 160.655 101.26) (width 0.1524) (layer F.Cu) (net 24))
 (segment (start 133.985 95.039) (end 133.985 91.44) (width 0.254) (layer B.Cu) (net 3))
 (segment (start 133.985 91.44) (end 135.89 89.535) (width 0.254) (layer B.Cu) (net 3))
 (segment (start 135.89 89.535) (end 135.89 88.56) (width 0.254) (layer B.Cu) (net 3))
 (segment (start 160.655 95.039) (end 160.655 94.185) (width 0.254) (layer B.Cu) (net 3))
 (segment (start 160.655 94.185) (end 159.766 93.296) (width 0.254) (layer B.Cu) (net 3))
 (segment (start 159.766 93.296) (end 159.766 90.142) (width 0.254) (layer B.Cu) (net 3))
 (segment (start 159.766 90.142) (end 158.184 88.56) (width 0.254) (layer B.Cu) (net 3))
 (segment (start 158.184 88.56) (end 157.48 88.56) (width 0.254) (layer B.Cu) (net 3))
 (segment (start 137.795 97.155) (end 135.951 97.155) (width 0.254) (layer B.Cu) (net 3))
 (segment (start 135.951 97.155) (end 133.985 95.189) (width 0.254) (layer B.Cu) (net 3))
 (segment (start 133.985 95.189) (end 133.985 95.039) (width 0.254) (layer B.Cu) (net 3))
 (segment (start 156.845 97.155) (end 158.689 97.155) (width 0.254) (layer B.Cu) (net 3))
 (segment (start 158.689 97.155) (end 160.655 95.189) (width 0.254) (layer B.Cu) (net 3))
 (segment (start 160.655 95.189) (end 160.655 95.039) (width 0.254) (layer B.Cu) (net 3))
 (segment (start 154.305 97.155) (end 156.845 97.155) (width 0.254) (layer F.Cu) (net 3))
 (segment (start 157.48 88.56) (end 155.575 88.56) (width 0.254) (layer B.Cu) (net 3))
 (segment (start 146.05 98.425) (end 147.230201 99.605201) (width 0.254) (layer B.Cu) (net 3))
 (segment (start 147.230201 99.605201) (end 150.750799 99.605201) (width 0.254) (layer B.Cu) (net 3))
 (segment (start 150.750799 99.605201) (end 153.201 97.155) (width 0.254) (layer B.Cu) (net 3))
 (segment (start 153.201 97.155) (end 154.305 97.155) (width 0.254) (layer B.Cu) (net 3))
 (segment (start 146.685 94.615) (end 146.685 97.79) (width 0.254) (layer B.Cu) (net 3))
 (segment (start 146.685 97.79) (end 146.05 98.425) (width 0.254) (layer B.Cu) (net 3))
 (segment (start 137.795 97.155) (end 140.335 97.155) (width 0.254) (layer B.Cu) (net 3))
 (segment (start 146.685 94.615) (end 146.685 93.055) (width 0.254) (layer B.Cu) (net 3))
 (segment (start 146.685 93.055) (end 145.705 92.075) (width 0.254) (layer B.Cu) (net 3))
 (segment (start 145.705 92.075) (end 145.255 92.075) (width 0.254) (layer B.Cu) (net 3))
 (segment (start 145.255 92.075) (end 143.065 92.075) (width 0.254) (layer B.Cu) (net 3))
 (segment (start 143.065 92.075) (end 139.7 88.71) (width 0.254) (layer B.Cu) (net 3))
 (segment (start 139.7 88.71) (end 139.7 88.56) (width 0.254) (layer B.Cu) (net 3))
 (segment (start 137.795 88.56) (end 139.7 88.56) (width 0.254) (layer B.Cu) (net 3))
 (segment (start 135.89 88.56) (end 137.795 88.56) (width 0.254) (layer B.Cu) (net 3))
 (segment (start 156.845 102.235) (end 155.485201 100.875201) (width 0.254) (layer B.Cu) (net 17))
 (segment (start 155.485201 100.875201) (end 155.485201 96.040839) (width 0.254) (layer B.Cu) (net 17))
 (segment (start 151.659 92.075) (end 150.655 92.075) (width 0.254) (layer B.Cu) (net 17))
 (segment (start 155.485201 96.040839) (end 155.075362 95.631) (width 0.254) (layer B.Cu) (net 17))
 (segment (start 155.075362 95.631) (end 152.527 95.631) (width 0.254) (layer B.Cu) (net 17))
 (segment (start 152.04 95.144) (end 152.04 92.456) (width 0.254) (layer B.Cu) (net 17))
 (segment (start 152.527 95.631) (end 152.04 95.144) (width 0.254) (layer B.Cu) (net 17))
 (segment (start 152.04 92.456) (end 151.659 92.075) (width 0.254) (layer B.Cu) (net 17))
 (segment (start 154.305 102.235) (end 156.845 102.235) (width 0.254) (layer B.Cu) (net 17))
 (segment (start 146.05 100.965) (end 147.32 102.235) (width 0.254) (layer B.Cu) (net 17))
 (segment (start 147.32 102.235) (end 154.305 102.235) (width 0.254) (layer B.Cu) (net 17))
 (segment (start 140.335 102.235) (end 137.795 102.235) (width 0.254) (layer B.Cu) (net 17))
 (segment (start 146.05 100.965) (end 141.605 100.965) (width 0.254) (layer B.Cu) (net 17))
 (segment (start 141.605 100.965) (end 140.335 102.235) (width 0.254) (layer B.Cu) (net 17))
 (segment (start 148.59 98.425) (end 148.59 97.222919) (width 0.1524) (layer B.Cu) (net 4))
 (segment (start 148.59 97.222919) (end 147.564401 96.19732) (width 0.1524) (layer B.Cu) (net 4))
 (segment (start 147.564401 96.19732) (end 147.564401 92.664401) (width 0.1524) (layer B.Cu) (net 4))
 (segment (start 147.564401 92.664401) (end 145.705 90.805) (width 0.1524) (layer B.Cu) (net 4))
 (segment (start 145.705 90.805) (end 145.255 90.805) (width 0.1524) (layer B.Cu) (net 4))
 (segment (start 150.114 98.171) (end 150.456899 97.828101) (width 0.1524) (layer B.Cu) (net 16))
 (segment (start 150.456899 97.828101) (end 150.456899 93.429821) (width 0.1524) (layer B.Cu) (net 16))
 (segment (start 150.456899 93.429821) (end 149.625599 92.598521) (width 0.1524) (layer B.Cu) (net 16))
 (segment (start 149.625599 92.598521) (end 149.625599 91.384401) (width 0.1524) (layer B.Cu) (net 16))
 (segment (start 149.625599 91.384401) (end 150.205 90.805) (width 0.1524) (layer B.Cu) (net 16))
 (segment (start 150.205 90.805) (end 150.655 90.805) (width 0.1524) (layer B.Cu) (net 16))
 (segment (start 148.59 100.965) (end 150.114 99.441) (width 0.1524) (layer F.Cu) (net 16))
 (segment (start 150.114 99.441) (end 150.114 98.171) (width 0.1524) (layer F.Cu) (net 16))
 (via (at 150.114 98.171) (size 0.6858) (drill 0.3302) (layers F.Cu B.Cu) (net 16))
 (segment (start 141.986 89.511933) (end 141.986 97.175514) (width 0.1524) (layer F.Cu) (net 8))
 (segment (start 141.986 97.175514) (end 140.545115 98.616399) (width 0.1524) (layer F.Cu) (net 8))
 (segment (start 140.545115 98.616399) (end 139.876001 98.616399) (width 0.1524) (layer F.Cu) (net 8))
 (segment (start 139.876001 98.616399) (end 138.7974 99.695) (width 0.1524) (layer F.Cu) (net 8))
 (segment (start 138.7974 99.695) (end 137.795 99.695) (width 0.1524) (layer F.Cu) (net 8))
 (segment (start 146.558 84.455) (end 146.558 84.939933) (width 0.1524) (layer F.Cu) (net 8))
 (segment (start 146.558 84.939933) (end 141.986 89.511933) (width 0.1524) (layer F.Cu) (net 8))
 (segment (start 145.255 84.455) (end 146.558 84.455) (width 0.1524) (layer B.Cu) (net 8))
 (via (at 146.558 84.455) (size 0.6858) (drill 0.3302) (layers F.Cu B.Cu) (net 8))
 (segment (start 146.711999 85.217) (end 146.584999 85.344) (width 0.1524) (layer F.Cu) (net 11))
 (segment (start 146.584999 85.344) (end 142.29081 89.638189) (width 0.1524) (layer F.Cu) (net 11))
 (segment (start 148.463 84.201) (end 147.727999 84.201) (width 0.1524) (layer F.Cu) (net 11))
 (segment (start 147.727999 84.201) (end 146.584999 85.344) (width 0.1524) (layer F.Cu) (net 11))
 (segment (start 150.655 84.455) (end 148.717 84.455) (width 0.1524) (layer B.Cu) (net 11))
 (segment (start 148.717 84.455) (end 148.463 84.201) (width 0.1524) (layer B.Cu) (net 11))
 (via (at 148.463 84.201) (size 0.6858) (drill 0.3302) (layers F.Cu B.Cu) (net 11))
 (segment (start 147.473999 84.455) (end 146.711999 85.217) (width 0.1524) (layer F.Cu) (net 11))
 (segment (start 150.655 84.455) (end 150.205 84.455) (width 0.1524) (layer B.Cu) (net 11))
 (segment (start 146.9025 85.026499) (end 146.711999 85.217) (width 0.1524) (layer F.Cu) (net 11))
 (segment (start 142.29081 89.638189) (end 142.29081 97.30177) (width 0.1524) (layer F.Cu) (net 11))
 (segment (start 142.29081 97.30177) (end 141.184999 98.407581) (width 0.1524) (layer F.Cu) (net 11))
 (segment (start 141.184999 98.845001) (end 140.335 99.695) (width 0.1524) (layer F.Cu) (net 11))
 (segment (start 141.184999 98.407581) (end 141.184999 98.845001) (width 0.1524) (layer F.Cu) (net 11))
 (segment (start 151.257 84.277934) (end 151.257 84.582) (width 0.1524) (layer F.Cu) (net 10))
 (segment (start 151.257 84.582) (end 151.257 84.963) (width 0.1524) (layer F.Cu) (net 10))
 (segment (start 151.13 82.296) (end 151.13 82.780933) (width 0.1524) (layer F.Cu) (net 10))
 (segment (start 151.13 82.780933) (end 151.257 82.907933) (width 0.1524) (layer F.Cu) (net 10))
 (segment (start 151.257 82.907933) (end 151.257 84.582) (width 0.1524) (layer F.Cu) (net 10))
 (segment (start 151.257 84.963) (end 151.257 97.6494) (width 0.1524) (layer F.Cu) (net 10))
 (segment (start 150.655 83.185) (end 150.655 82.771) (width 0.1524) (layer B.Cu) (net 10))
 (segment (start 150.655 82.771) (end 151.13 82.296) (width 0.1524) (layer B.Cu) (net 10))
 (via (at 151.13 82.296) (size 0.6858) (drill 0.3302) (layers F.Cu B.Cu) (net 10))
 (segment (start 151.257 97.6494) (end 153.3026 99.695) (width 0.1524) (layer F.Cu) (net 10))
 (segment (start 153.3026 99.695) (end 154.305 99.695) (width 0.1524) (layer F.Cu) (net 10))
 (segment (start 147.256501 83.756501) (end 148.102321 83.756501) (width 0.1524) (layer F.Cu) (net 9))
 (segment (start 148.673822 83.185) (end 149.733 83.185) (width 0.1524) (layer F.Cu) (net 9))
 (segment (start 148.102321 83.756501) (end 148.673822 83.185) (width 0.1524) (layer F.Cu) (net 9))
 (segment (start 149.733 83.185) (end 150.95219 84.40419) (width 0.1524) (layer F.Cu) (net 9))
 (segment (start 150.95219 84.40419) (end 150.95219 98.453672) (width 0.1524) (layer F.Cu) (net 9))
 (segment (start 150.95219 98.453672) (end 153.272119 100.773601) (width 0.1524) (layer F.Cu) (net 9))
 (segment (start 153.272119 100.773601) (end 155.766399 100.773601) (width 0.1524) (layer F.Cu) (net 9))
 (segment (start 155.766399 100.773601) (end 156.845 99.695) (width 0.1524) (layer F.Cu) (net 9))
 (segment (start 145.255 83.185) (end 146.685 83.185) (width 0.1524) (layer B.Cu) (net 9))
 (segment (start 146.685 83.185) (end 147.256501 83.756501) (width 0.1524) (layer B.Cu) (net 9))
 (via (at 147.256501 83.756501) (size 0.6858) (drill 0.3302) (layers F.Cu B.Cu) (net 9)))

